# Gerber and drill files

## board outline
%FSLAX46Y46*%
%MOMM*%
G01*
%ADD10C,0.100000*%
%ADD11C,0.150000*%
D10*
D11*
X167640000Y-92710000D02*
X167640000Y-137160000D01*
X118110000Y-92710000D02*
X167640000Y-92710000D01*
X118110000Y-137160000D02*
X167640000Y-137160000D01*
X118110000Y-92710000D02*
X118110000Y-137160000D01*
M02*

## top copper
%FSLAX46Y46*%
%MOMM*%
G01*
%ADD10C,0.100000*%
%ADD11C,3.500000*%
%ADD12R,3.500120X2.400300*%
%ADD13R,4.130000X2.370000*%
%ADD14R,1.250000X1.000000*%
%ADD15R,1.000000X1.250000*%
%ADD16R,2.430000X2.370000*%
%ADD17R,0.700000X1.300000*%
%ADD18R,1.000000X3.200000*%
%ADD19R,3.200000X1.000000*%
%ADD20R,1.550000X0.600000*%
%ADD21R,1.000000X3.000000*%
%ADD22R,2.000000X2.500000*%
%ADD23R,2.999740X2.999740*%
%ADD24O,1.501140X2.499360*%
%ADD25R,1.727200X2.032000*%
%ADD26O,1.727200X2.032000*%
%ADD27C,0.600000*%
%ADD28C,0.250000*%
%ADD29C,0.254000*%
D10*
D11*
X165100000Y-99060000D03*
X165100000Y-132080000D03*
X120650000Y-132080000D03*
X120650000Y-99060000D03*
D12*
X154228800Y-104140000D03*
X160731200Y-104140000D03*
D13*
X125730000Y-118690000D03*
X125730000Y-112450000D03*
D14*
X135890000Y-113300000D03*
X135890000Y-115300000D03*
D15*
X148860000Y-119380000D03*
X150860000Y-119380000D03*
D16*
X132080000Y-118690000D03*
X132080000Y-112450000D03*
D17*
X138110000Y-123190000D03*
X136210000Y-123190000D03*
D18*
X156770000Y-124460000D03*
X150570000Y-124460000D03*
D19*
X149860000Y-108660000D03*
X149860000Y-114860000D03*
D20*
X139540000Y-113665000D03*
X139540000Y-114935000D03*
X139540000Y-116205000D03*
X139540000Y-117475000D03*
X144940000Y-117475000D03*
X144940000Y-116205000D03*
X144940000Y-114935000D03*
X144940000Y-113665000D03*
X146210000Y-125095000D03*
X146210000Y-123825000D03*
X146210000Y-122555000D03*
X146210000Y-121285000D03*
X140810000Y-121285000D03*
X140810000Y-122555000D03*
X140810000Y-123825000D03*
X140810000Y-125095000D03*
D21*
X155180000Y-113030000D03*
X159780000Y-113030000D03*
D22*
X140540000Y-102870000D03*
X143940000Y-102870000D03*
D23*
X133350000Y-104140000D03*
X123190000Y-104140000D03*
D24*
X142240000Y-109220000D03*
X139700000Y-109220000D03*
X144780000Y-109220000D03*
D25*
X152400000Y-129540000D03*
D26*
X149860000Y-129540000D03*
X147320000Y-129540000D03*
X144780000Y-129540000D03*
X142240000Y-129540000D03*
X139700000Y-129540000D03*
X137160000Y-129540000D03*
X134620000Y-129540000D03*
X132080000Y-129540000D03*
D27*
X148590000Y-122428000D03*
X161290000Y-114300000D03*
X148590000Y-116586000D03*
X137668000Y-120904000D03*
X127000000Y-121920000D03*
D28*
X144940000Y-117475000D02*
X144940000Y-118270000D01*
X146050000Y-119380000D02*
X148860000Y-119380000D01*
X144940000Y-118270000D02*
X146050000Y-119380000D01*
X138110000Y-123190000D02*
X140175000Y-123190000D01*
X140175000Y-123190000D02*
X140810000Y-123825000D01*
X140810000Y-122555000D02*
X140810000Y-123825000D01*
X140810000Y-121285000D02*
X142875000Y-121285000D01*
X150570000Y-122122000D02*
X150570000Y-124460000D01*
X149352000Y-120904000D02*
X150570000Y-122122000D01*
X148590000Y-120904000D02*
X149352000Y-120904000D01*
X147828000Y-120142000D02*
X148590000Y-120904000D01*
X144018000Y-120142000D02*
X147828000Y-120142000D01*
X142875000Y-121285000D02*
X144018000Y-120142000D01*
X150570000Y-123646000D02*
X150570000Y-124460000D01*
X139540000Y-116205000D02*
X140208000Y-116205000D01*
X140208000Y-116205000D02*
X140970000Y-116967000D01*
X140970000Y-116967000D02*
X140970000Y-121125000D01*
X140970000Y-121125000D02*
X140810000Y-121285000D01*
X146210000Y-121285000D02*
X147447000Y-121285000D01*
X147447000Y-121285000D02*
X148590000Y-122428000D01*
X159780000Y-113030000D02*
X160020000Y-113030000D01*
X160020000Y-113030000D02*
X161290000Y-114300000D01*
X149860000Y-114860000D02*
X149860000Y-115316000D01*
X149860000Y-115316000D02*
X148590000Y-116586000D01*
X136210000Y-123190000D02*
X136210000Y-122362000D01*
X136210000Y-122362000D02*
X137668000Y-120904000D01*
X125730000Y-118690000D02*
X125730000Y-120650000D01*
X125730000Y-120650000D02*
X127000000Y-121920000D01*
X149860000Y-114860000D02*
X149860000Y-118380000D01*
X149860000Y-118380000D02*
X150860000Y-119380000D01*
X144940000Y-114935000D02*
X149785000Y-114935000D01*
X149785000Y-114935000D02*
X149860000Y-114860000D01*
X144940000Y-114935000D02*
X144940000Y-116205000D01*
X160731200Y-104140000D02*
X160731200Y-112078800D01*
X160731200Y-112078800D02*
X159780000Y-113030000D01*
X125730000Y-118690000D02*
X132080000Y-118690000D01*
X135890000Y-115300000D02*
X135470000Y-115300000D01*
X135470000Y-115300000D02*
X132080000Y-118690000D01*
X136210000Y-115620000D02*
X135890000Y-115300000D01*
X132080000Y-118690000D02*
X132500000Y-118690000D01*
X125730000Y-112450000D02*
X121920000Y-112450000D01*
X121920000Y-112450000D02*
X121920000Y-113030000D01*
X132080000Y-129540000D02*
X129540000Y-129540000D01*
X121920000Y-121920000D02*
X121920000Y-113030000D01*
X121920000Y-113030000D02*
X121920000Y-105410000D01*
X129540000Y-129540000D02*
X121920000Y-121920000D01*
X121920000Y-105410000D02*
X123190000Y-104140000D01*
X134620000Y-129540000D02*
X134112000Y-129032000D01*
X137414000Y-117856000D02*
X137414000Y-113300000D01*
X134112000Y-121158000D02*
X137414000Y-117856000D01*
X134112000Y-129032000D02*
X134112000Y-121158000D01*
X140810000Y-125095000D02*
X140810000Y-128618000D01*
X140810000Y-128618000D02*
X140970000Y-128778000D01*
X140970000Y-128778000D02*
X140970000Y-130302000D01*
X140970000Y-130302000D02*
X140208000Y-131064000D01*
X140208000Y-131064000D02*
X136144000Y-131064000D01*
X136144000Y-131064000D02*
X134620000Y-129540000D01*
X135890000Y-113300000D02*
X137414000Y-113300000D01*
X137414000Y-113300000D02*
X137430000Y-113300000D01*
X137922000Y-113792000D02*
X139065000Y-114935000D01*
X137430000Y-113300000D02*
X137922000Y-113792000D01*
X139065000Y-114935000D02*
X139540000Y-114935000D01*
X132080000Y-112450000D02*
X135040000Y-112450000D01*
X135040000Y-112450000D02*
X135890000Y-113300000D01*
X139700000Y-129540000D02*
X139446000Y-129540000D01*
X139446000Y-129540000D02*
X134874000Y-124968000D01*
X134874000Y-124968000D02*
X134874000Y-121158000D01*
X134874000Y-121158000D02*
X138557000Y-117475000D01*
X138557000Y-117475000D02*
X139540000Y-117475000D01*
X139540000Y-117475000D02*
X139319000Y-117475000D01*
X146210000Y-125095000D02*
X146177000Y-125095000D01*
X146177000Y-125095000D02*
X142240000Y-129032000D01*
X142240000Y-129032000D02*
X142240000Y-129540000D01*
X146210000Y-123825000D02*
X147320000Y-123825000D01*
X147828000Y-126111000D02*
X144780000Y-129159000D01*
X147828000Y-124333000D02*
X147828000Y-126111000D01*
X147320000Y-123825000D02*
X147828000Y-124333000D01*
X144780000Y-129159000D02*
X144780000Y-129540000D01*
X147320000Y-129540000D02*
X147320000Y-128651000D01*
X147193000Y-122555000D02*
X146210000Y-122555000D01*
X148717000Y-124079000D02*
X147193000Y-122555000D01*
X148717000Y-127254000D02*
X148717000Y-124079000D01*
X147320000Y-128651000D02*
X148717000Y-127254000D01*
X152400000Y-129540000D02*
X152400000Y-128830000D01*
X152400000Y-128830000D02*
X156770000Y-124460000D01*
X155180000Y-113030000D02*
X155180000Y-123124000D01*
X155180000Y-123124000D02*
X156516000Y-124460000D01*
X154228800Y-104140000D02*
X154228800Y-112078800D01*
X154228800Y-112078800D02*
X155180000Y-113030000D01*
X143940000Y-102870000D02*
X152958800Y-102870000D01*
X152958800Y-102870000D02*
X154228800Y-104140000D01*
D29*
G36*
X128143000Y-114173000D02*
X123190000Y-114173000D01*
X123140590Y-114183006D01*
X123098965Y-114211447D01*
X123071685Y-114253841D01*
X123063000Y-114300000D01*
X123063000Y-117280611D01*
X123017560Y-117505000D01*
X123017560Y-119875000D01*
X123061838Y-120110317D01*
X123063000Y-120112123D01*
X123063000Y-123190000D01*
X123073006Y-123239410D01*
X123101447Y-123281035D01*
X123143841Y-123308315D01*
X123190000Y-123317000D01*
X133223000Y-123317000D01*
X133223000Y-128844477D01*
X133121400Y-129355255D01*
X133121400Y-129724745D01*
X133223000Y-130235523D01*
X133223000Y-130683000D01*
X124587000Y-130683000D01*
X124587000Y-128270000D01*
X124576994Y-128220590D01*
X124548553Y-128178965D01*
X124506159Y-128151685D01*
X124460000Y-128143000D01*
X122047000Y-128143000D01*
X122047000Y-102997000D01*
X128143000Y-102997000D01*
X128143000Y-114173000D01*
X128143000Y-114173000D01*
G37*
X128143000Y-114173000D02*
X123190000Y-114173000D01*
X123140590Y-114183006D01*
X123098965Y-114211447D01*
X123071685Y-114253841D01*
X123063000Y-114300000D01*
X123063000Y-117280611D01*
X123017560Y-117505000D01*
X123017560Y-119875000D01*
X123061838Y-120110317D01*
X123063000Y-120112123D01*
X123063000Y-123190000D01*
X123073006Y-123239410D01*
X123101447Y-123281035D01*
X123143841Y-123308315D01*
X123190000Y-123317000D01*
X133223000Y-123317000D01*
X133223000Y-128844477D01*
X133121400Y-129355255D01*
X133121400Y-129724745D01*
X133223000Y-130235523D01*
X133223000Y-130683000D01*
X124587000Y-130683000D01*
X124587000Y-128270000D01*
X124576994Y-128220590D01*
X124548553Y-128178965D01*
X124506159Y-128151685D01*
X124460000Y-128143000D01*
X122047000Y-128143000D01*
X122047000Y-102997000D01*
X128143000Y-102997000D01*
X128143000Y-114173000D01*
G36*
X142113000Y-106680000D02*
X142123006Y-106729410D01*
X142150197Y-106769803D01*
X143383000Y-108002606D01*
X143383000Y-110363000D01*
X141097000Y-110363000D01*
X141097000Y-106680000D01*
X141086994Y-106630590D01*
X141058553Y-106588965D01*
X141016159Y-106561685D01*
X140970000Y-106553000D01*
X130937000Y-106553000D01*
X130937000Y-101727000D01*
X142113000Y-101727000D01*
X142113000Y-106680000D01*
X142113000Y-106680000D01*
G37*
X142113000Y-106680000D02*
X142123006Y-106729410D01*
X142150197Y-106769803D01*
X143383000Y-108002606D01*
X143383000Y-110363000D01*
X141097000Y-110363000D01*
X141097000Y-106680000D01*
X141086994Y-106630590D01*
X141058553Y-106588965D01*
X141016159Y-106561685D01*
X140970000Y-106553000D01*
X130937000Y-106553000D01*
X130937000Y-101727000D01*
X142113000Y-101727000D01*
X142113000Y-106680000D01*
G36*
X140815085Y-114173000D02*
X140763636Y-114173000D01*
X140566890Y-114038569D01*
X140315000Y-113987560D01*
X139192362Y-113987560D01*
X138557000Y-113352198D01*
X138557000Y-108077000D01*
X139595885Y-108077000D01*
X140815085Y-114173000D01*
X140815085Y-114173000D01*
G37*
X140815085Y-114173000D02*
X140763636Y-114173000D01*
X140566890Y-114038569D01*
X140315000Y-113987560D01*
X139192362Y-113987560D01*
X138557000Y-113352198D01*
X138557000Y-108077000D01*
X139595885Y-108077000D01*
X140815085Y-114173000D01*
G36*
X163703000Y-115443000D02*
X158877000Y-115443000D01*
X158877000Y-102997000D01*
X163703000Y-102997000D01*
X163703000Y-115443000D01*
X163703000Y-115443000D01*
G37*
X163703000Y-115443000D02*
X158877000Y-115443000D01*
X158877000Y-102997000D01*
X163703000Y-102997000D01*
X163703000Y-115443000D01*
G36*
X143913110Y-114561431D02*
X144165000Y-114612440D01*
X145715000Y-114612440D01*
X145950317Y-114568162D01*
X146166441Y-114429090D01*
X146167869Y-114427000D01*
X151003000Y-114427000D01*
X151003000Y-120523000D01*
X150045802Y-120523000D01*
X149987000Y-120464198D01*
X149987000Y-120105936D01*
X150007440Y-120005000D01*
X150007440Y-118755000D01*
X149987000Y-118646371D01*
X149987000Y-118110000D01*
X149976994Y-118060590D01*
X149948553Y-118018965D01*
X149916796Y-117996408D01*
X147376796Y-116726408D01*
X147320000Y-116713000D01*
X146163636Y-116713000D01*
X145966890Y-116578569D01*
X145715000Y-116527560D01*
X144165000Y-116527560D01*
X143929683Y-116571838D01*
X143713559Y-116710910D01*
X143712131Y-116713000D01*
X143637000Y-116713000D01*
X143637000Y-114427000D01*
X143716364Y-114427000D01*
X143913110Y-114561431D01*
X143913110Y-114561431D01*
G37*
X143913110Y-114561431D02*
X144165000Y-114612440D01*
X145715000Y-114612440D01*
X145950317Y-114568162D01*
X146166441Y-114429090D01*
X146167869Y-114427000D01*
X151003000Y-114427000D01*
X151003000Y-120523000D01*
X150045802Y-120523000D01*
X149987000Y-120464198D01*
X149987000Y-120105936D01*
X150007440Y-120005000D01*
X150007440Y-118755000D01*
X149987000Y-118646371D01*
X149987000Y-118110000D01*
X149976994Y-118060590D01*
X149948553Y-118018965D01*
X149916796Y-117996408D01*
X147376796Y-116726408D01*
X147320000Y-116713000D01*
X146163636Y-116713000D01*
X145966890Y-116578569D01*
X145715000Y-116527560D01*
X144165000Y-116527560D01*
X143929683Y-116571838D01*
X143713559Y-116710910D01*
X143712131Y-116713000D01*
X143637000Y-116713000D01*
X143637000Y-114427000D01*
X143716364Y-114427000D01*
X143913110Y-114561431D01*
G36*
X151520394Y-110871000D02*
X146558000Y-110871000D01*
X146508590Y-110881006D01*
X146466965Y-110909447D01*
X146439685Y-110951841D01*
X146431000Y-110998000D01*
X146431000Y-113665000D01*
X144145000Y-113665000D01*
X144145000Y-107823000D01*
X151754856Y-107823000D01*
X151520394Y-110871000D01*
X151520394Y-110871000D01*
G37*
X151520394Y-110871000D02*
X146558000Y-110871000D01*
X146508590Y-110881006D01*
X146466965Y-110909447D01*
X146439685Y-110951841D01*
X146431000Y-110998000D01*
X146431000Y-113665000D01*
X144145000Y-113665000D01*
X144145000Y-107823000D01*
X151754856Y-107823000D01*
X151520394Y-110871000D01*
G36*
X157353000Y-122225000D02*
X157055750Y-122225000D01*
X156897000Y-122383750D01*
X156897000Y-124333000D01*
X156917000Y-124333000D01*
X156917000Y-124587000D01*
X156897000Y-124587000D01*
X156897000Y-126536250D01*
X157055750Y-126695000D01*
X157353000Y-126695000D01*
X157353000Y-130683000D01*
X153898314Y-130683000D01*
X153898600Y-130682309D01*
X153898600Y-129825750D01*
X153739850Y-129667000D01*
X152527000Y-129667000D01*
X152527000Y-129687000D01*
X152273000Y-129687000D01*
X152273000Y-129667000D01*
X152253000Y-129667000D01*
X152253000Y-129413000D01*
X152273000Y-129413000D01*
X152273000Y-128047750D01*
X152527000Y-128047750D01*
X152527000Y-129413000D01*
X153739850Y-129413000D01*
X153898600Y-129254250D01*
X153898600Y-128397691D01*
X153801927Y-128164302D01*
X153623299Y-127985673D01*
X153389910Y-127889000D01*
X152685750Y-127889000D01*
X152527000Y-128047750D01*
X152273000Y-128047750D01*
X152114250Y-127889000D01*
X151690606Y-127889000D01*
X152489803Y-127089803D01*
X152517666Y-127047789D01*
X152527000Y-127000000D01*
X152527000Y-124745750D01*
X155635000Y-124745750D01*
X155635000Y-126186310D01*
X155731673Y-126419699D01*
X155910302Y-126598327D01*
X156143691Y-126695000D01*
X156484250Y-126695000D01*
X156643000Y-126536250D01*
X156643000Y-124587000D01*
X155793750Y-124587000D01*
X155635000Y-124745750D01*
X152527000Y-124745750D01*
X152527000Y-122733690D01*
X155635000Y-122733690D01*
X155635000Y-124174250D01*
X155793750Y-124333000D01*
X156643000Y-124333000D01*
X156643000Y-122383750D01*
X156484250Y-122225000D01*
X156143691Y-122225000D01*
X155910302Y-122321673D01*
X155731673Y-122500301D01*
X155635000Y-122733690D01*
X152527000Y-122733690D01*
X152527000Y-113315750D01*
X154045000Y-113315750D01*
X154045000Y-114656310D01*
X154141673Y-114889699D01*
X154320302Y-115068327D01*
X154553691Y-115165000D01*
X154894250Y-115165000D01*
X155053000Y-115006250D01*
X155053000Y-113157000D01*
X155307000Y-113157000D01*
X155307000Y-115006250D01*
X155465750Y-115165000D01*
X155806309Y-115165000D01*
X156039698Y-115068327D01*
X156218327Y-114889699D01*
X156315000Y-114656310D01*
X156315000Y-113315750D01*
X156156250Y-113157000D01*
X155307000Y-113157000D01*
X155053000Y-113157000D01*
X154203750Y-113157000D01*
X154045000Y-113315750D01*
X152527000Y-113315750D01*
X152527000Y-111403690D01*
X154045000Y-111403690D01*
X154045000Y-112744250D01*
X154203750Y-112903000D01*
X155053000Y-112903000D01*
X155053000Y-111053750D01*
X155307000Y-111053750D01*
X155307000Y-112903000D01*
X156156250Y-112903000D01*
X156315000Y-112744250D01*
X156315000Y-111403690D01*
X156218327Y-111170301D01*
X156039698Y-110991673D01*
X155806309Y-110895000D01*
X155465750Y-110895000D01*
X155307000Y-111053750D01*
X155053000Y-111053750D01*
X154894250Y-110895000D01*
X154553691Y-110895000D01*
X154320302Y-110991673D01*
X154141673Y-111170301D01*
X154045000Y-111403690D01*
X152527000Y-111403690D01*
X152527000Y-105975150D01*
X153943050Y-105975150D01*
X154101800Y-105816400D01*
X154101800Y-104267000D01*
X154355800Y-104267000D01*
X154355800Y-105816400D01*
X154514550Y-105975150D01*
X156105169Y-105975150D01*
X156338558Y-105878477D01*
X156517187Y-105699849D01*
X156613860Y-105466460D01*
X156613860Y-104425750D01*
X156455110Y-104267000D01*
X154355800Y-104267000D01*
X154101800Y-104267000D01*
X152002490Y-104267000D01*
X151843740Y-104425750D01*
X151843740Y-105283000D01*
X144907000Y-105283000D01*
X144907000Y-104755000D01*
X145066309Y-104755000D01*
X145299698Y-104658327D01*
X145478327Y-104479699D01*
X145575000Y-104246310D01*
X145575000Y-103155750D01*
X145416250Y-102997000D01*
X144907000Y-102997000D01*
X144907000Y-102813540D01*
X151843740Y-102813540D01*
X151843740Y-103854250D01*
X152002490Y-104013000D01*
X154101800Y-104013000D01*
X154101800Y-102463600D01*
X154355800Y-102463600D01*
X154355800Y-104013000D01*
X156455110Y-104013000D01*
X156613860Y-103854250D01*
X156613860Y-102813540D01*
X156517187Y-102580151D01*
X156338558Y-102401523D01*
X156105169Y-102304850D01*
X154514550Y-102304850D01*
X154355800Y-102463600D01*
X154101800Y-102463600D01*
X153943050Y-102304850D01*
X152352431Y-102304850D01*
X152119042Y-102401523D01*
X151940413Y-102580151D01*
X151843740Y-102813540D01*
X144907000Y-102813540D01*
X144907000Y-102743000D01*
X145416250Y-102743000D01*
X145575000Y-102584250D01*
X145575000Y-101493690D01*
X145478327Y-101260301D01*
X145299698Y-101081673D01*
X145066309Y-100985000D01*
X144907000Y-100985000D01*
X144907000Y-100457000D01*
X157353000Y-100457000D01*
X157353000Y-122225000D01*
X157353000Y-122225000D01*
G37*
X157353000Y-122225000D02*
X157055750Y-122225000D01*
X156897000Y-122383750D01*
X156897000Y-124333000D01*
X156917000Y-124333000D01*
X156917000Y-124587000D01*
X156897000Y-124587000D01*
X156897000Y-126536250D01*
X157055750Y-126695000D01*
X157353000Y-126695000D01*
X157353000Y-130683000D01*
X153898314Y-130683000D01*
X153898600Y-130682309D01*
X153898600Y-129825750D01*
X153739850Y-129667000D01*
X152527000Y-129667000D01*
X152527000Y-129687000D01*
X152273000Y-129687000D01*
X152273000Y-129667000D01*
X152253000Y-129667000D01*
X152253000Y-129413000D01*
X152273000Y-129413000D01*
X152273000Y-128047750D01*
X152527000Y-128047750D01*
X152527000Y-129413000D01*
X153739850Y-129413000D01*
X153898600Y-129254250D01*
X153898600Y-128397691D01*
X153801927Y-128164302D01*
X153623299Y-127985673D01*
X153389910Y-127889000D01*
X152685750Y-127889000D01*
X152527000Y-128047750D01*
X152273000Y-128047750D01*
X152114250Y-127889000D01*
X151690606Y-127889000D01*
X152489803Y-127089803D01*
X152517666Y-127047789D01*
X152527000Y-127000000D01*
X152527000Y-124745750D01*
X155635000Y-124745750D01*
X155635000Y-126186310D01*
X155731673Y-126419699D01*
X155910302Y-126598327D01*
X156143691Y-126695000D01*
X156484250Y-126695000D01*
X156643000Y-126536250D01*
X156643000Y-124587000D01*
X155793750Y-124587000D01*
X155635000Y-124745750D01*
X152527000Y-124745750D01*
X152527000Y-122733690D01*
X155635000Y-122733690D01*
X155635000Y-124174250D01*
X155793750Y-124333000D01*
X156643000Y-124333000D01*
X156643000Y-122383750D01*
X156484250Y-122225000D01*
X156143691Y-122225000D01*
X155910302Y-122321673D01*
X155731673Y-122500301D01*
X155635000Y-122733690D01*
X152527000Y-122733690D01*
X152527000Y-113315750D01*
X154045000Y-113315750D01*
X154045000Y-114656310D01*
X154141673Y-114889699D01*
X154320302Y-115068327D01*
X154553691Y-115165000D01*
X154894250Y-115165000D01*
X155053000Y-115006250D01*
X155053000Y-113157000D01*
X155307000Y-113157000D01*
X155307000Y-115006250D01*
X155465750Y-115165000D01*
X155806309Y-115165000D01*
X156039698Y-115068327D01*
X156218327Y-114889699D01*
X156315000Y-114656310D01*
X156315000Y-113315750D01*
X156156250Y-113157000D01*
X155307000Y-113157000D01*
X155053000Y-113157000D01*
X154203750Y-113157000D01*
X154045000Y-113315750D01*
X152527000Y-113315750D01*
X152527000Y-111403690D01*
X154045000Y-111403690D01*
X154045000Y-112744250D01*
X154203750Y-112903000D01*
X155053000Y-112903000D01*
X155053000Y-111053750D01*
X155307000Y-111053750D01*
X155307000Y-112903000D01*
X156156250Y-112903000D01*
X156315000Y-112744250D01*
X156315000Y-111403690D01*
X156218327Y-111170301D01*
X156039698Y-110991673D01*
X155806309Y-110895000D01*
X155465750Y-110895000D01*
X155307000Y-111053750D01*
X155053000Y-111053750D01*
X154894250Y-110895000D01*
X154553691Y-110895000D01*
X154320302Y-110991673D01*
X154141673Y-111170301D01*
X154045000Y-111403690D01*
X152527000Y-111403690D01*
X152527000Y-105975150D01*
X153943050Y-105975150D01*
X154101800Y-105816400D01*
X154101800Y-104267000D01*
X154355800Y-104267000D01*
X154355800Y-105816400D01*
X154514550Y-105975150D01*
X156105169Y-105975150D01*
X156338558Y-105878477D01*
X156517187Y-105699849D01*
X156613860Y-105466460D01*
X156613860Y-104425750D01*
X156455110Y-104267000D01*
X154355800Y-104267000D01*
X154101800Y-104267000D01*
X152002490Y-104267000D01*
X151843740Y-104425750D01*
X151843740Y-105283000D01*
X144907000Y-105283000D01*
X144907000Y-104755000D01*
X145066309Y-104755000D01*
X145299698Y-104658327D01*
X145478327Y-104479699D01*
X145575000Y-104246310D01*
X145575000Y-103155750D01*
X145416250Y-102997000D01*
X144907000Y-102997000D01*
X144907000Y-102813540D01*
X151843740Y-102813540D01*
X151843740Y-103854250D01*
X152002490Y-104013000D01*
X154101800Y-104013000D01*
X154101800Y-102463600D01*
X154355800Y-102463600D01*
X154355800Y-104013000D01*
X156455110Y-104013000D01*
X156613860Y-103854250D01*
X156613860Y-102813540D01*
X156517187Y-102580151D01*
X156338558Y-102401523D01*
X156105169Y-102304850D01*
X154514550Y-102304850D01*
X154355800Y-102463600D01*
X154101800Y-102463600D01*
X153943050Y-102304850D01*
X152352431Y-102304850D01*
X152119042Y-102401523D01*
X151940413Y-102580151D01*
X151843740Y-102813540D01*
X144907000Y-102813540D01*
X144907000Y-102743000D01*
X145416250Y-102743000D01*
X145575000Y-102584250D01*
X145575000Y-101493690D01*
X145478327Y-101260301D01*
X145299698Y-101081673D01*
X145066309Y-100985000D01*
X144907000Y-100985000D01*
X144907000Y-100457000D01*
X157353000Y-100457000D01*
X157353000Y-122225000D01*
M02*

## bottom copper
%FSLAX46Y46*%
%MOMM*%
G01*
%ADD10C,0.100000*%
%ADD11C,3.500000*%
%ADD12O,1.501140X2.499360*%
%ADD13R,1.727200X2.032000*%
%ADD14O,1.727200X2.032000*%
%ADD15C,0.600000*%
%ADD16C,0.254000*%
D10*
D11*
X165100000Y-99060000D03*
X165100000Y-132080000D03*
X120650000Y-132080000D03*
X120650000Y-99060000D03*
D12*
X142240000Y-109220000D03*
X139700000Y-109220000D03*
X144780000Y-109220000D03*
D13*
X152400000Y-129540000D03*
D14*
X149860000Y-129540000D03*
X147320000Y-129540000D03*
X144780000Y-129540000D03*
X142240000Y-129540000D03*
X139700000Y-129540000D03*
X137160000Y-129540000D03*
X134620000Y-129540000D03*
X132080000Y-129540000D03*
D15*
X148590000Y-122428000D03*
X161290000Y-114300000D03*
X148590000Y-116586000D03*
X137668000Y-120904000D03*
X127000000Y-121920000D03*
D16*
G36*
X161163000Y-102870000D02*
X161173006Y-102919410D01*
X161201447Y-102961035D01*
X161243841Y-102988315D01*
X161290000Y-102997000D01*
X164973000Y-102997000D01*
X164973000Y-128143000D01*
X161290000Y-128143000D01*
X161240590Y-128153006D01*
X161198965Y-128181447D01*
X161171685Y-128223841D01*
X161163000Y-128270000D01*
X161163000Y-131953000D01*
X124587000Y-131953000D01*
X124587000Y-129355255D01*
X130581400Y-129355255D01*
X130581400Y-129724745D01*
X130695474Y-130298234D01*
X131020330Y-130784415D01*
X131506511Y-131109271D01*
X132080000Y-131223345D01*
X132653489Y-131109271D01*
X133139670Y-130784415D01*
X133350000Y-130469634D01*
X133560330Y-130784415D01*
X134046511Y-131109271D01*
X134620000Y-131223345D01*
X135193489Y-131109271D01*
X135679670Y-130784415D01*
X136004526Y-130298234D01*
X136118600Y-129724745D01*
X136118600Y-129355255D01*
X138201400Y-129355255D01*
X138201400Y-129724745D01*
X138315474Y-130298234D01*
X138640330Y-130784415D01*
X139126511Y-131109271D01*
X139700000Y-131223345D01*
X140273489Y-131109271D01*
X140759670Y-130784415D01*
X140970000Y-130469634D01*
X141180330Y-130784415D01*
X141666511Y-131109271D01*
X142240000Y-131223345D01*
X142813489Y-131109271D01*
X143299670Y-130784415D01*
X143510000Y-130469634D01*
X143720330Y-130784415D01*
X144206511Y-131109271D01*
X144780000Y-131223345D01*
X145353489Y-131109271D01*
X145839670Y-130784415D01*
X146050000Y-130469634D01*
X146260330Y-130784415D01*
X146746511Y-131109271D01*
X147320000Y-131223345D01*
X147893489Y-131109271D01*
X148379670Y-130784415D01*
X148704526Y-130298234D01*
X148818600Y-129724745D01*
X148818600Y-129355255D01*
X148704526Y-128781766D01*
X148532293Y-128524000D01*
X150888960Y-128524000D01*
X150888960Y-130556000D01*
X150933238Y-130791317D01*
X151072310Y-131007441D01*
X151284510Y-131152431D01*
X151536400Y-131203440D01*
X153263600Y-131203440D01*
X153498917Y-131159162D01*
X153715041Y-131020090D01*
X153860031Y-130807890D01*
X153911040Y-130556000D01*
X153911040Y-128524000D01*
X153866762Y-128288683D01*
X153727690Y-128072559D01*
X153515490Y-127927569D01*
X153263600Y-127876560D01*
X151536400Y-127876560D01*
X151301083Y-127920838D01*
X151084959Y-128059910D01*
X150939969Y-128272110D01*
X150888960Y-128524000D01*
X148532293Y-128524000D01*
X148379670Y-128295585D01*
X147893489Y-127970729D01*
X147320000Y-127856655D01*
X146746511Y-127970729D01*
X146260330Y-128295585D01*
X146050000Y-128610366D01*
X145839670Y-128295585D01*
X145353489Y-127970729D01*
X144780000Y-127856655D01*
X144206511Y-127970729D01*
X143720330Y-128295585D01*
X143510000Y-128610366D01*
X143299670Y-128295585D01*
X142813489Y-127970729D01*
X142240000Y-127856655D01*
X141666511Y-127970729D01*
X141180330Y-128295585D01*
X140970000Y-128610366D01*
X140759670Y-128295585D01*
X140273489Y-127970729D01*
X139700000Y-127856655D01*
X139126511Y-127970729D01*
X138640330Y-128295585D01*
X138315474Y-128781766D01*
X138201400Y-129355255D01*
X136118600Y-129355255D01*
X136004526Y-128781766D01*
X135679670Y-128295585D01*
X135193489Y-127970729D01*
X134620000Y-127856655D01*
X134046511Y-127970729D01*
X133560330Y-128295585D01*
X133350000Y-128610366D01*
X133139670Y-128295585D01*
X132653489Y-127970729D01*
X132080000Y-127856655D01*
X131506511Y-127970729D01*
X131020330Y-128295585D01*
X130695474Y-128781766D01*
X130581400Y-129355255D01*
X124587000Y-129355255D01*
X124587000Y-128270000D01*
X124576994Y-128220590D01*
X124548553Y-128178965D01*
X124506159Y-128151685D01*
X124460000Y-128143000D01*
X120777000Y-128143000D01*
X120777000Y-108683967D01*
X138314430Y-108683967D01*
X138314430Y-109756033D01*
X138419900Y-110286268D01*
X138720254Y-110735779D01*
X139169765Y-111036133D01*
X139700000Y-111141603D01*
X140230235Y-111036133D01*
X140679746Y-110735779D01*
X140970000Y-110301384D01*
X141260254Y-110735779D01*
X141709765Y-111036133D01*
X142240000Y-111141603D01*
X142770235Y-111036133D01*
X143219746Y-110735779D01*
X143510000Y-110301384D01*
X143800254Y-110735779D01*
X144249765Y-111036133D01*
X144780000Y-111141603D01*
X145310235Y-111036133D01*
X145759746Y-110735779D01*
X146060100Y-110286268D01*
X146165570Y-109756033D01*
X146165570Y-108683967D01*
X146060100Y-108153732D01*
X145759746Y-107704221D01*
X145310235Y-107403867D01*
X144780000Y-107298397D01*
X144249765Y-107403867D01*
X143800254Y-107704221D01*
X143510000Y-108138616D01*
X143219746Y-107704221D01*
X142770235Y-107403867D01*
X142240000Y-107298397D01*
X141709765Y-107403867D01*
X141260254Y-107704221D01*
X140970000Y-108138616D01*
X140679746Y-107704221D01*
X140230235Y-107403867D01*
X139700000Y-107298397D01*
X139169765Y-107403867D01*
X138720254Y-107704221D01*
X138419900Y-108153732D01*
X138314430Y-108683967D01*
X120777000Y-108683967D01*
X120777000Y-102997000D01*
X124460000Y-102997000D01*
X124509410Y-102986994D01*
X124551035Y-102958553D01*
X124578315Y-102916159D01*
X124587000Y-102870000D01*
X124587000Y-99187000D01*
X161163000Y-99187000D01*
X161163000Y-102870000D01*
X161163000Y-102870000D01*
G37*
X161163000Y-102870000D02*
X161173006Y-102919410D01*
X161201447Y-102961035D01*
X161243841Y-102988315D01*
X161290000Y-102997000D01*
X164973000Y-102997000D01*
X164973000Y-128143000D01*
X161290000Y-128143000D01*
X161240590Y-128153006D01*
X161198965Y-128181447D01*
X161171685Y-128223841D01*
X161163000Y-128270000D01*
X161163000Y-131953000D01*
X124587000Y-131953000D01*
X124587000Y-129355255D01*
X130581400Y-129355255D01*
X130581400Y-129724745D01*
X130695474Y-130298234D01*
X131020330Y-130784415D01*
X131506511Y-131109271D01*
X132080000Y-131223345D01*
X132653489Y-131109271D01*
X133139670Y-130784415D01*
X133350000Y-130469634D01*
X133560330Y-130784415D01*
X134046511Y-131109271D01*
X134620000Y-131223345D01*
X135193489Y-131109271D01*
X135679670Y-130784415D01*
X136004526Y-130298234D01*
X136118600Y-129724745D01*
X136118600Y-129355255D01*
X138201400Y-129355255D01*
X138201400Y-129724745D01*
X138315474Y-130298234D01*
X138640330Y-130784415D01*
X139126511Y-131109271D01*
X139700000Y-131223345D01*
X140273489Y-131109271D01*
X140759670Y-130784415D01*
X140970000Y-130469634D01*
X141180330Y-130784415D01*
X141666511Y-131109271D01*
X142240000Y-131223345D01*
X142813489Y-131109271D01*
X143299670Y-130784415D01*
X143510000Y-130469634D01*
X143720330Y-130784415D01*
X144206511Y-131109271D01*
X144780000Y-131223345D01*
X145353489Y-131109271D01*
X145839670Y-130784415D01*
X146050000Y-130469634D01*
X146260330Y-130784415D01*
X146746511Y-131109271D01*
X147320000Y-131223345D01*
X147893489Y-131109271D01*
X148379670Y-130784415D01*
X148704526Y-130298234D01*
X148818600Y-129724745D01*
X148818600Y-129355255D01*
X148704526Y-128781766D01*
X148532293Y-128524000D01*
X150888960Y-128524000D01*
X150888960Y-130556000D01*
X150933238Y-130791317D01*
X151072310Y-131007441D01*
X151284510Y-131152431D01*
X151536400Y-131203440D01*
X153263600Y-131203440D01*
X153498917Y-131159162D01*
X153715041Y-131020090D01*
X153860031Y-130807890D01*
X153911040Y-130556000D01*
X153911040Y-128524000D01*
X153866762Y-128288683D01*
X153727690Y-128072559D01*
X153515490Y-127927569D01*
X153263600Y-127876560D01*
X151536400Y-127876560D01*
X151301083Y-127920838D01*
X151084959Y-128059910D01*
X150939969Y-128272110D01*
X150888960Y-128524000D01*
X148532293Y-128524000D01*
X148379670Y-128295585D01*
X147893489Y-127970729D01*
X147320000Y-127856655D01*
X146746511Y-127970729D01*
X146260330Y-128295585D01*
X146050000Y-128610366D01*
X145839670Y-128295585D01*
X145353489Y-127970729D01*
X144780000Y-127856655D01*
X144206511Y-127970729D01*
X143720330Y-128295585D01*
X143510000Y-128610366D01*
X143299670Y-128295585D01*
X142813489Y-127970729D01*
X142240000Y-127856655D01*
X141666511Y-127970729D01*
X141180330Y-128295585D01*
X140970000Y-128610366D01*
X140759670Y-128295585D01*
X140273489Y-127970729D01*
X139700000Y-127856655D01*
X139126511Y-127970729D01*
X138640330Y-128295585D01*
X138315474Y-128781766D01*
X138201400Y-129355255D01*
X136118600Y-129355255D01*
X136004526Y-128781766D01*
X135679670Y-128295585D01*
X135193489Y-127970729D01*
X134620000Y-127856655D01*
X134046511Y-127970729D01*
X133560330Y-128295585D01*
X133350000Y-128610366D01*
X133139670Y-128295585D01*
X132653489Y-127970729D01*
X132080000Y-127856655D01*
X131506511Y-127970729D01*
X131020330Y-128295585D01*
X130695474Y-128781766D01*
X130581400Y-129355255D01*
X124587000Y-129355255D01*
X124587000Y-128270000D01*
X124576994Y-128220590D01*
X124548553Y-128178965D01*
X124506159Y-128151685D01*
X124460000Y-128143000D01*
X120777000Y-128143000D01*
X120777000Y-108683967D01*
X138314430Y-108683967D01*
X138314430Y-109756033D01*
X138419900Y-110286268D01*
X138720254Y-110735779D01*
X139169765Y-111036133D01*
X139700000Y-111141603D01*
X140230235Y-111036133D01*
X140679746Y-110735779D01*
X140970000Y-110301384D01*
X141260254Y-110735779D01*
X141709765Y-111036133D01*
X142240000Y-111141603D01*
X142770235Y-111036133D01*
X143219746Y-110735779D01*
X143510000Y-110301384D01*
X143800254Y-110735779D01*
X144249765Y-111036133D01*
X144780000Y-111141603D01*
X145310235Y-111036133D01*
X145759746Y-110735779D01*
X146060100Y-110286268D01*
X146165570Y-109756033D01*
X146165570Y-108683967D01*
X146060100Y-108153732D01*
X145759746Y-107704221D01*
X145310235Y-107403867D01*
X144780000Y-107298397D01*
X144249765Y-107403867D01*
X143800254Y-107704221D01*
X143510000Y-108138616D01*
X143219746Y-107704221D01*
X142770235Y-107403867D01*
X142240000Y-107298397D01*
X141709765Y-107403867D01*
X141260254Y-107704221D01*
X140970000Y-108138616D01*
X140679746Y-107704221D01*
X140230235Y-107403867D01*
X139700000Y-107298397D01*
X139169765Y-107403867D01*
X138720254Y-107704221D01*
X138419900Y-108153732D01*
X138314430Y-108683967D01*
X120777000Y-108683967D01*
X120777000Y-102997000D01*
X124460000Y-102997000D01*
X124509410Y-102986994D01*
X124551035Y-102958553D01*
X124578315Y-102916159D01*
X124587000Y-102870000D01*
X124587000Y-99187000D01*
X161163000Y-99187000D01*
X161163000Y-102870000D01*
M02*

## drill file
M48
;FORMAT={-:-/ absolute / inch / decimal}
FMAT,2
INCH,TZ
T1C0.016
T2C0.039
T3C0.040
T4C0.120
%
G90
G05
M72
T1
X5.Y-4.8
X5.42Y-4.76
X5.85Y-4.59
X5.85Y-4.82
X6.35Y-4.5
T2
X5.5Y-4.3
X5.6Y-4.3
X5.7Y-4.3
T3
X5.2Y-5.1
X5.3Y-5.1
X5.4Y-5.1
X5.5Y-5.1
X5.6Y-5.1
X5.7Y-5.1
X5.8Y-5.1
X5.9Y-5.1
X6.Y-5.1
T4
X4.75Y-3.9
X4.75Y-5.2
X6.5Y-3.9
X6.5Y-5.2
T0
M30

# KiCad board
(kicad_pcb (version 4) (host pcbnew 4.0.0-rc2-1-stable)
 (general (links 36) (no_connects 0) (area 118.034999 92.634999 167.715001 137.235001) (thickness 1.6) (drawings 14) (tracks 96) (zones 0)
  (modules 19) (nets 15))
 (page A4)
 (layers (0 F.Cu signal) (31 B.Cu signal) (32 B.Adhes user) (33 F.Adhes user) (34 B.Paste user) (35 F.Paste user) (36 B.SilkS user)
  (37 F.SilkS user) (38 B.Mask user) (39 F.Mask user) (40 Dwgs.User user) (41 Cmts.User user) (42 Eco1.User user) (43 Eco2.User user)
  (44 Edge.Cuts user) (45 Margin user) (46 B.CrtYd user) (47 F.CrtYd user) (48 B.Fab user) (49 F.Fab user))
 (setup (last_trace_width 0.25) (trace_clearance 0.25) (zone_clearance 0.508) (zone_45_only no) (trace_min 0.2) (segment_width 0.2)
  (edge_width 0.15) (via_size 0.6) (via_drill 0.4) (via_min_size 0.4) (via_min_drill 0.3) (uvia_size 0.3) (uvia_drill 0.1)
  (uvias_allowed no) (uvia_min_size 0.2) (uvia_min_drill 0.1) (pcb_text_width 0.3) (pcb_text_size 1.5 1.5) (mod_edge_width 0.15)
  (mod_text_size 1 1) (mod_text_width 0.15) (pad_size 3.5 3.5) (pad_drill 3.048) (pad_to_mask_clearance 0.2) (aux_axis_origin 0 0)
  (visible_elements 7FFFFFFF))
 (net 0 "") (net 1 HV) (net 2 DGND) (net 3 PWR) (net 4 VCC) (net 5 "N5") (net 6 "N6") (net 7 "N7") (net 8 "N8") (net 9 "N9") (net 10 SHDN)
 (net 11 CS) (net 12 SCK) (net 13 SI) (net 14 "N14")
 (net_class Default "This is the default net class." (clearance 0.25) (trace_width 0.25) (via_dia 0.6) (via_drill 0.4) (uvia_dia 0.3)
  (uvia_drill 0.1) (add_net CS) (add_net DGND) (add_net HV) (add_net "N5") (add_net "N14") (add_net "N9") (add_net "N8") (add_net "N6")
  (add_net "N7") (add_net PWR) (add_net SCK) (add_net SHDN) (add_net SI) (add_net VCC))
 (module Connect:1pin (layer F.Cu) (at 165.1 99.06)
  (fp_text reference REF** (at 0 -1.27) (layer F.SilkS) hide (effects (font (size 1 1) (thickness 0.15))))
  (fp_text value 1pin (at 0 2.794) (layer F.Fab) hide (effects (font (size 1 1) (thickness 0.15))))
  (pad 1 thru_hole circle (at 0 0) (size 3.5 3.5) (drill 3.048) (layers *.Cu *.Mask F.SilkS)))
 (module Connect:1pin (layer F.Cu) (at 165.1 132.08)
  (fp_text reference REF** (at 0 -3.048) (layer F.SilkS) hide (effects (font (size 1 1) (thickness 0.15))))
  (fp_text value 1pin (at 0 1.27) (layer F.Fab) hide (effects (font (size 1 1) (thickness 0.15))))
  (pad 1 thru_hole circle (at 0 0) (size 3.5 3.5) (drill 3.048) (layers *.Cu *.Mask F.SilkS)))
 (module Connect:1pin (layer F.Cu) (at 120.65 132.08)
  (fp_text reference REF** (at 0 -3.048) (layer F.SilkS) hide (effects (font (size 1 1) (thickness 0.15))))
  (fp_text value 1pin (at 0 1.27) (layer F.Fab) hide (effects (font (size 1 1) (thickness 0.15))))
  (pad 1 thru_hole circle (at 0 0) (size 3.5 3.5) (drill 3.048) (layers *.Cu *.Mask F.SilkS)))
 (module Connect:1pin (layer F.Cu) (at 120.65 99.06)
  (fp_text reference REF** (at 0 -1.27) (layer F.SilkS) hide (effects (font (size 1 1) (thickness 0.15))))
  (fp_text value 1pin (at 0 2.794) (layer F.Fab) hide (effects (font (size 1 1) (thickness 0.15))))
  (pad 1 thru_hole circle (at 0 0) (size 3.5 3.5) (drill 3.048) (layers *.Cu *.Mask F.SilkS)))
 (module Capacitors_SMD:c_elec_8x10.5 (layer F.Cu) (at 157.48 104.14 180)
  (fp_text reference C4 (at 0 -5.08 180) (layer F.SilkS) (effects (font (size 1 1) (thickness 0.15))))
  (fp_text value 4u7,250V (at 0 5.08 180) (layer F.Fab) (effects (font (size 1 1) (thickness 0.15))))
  (pad 1 smd rect (at 3.2512 0 180) (size 3.50012 2.4003) (layers F.Cu F.Paste F.Mask) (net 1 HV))
  (pad 2 smd rect (at -3.2512 0 180) (size 3.50012 2.4003) (layers F.Cu F.Paste F.Mask) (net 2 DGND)))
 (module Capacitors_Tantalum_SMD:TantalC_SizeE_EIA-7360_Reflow (layer F.Cu) (at 125.73 115.57 270)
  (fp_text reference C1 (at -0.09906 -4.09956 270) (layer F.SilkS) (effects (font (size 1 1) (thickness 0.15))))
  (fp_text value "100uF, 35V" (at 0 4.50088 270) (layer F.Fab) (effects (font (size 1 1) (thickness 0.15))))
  (pad 2 smd rect (at 3.12 0 270) (size 2.37 4.13) (layers F.Cu F.Paste F.Mask) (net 2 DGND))
  (pad 1 smd rect (at -3.12 0 270) (size 2.37 4.13) (layers F.Cu F.Paste F.Mask) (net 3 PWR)))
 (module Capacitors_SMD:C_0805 (layer F.Cu) (at 135.89 114.3 270)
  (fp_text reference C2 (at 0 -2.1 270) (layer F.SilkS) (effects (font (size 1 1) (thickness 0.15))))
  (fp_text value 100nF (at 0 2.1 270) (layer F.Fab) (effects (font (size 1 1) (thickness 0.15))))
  (pad 1 smd rect (at -1 0 270) (size 1 1.25) (layers F.Cu F.Paste F.Mask) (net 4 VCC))
  (pad 2 smd rect (at 1 0 270) (size 1 1.25) (layers F.Cu F.Paste F.Mask) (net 2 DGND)))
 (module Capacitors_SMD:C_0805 (layer F.Cu) (at 149.86 119.38)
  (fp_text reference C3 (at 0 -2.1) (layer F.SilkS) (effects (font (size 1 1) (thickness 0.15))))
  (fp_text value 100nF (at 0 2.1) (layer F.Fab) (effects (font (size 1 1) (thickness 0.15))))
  (pad 1 smd rect (at -1 0) (size 1 1.25) (layers F.Cu F.Paste F.Mask) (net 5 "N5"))
  (pad 2 smd rect (at 1 0) (size 1 1.25) (layers F.Cu F.Paste F.Mask) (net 2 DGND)))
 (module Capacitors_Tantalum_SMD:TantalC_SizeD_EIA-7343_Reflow (layer F.Cu) (at 132.08 115.57 270)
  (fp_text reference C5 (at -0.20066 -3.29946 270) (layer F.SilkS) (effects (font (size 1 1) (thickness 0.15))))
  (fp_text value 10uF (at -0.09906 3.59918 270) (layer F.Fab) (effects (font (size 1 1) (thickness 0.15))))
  (pad 2 smd rect (at 3.12 0 270) (size 2.37 2.43) (layers F.Cu F.Paste F.Mask) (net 2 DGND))
  (pad 1 smd rect (at -3.12 0 270) (size 2.37 2.43) (layers F.Cu F.Paste F.Mask) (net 4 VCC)))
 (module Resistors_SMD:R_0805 (layer F.Cu) (at 137.16 123.19 180)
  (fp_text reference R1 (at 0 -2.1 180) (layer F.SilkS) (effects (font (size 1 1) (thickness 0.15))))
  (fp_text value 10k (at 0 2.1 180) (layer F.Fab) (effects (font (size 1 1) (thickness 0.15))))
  (pad 1 smd rect (at -0.95 0 180) (size 0.7 1.3) (layers F.Cu F.Paste F.Mask) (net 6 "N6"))
  (pad 2 smd rect (at 0.95 0 180) (size 0.7 1.3) (layers F.Cu F.Paste F.Mask) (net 2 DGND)))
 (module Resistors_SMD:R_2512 (layer F.Cu) (at 153.67 124.46 180)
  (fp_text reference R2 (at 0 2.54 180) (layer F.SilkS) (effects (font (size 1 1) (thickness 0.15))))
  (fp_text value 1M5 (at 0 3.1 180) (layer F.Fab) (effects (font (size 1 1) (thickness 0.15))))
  (pad 1 smd rect (at -3.1 0 180) (size 1 3.2) (layers F.Cu F.Paste F.Mask) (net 1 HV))
  (pad 2 smd rect (at 3.1 0 180) (size 1 3.2) (layers F.Cu F.Paste F.Mask) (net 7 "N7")))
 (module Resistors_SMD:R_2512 (layer F.Cu) (at 149.86 111.76 270)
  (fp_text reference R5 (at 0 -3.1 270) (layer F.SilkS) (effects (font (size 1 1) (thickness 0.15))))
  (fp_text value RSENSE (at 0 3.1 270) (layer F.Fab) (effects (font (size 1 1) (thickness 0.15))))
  (pad 1 smd rect (at -3.1 0 270) (size 1 3.2) (layers F.Cu F.Paste F.Mask) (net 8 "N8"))
  (pad 2 smd rect (at 3.1 0 270) (size 1 3.2) (layers F.Cu F.Paste F.Mask) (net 2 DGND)))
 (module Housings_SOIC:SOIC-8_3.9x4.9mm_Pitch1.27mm (layer F.Cu) (at 142.24 115.57)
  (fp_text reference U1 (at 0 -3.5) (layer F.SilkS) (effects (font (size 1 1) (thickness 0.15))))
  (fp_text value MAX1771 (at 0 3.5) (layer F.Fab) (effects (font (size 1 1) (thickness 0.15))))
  (pad 1 smd rect (at -2.7 -1.905) (size 1.55 0.6) (layers F.Cu F.Paste F.Mask) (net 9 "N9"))
  (pad 2 smd rect (at -2.7 -0.635) (size 1.55 0.6) (layers F.Cu F.Paste F.Mask) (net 4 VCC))
  (pad 3 smd rect (at -2.7 0.635) (size 1.55 0.6) (layers F.Cu F.Paste F.Mask) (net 7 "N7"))
  (pad 4 smd rect (at -2.7 1.905) (size 1.55 0.6) (layers F.Cu F.Paste F.Mask) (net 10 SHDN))
  (pad 5 smd rect (at 2.7 1.905) (size 1.55 0.6) (layers F.Cu F.Paste F.Mask) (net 5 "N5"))
  (pad 6 smd rect (at 2.7 0.635) (size 1.55 0.6) (layers F.Cu F.Paste F.Mask) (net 2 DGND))
  (pad 7 smd rect (at 2.7 -0.635) (size 1.55 0.6) (layers F.Cu F.Paste F.Mask) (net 2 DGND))
  (pad 8 smd rect (at 2.7 -1.905) (size 1.55 0.6) (layers F.Cu F.Paste F.Mask) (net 8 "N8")))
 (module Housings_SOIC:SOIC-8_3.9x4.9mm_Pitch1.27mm (layer F.Cu) (at 143.51 123.19 180)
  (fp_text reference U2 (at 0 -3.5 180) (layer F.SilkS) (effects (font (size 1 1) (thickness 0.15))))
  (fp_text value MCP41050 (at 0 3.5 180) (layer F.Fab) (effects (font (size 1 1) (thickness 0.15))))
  (pad 1 smd rect (at -2.7 -1.905 180) (size 1.55 0.6) (layers F.Cu F.Paste F.Mask) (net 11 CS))
  (pad 2 smd rect (at -2.7 -0.635 180) (size 1.55 0.6) (layers F.Cu F.Paste F.Mask) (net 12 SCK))
  (pad 3 smd rect (at -2.7 0.635 180) (size 1.55 0.6) (layers F.Cu F.Paste F.Mask) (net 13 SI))
  (pad 4 smd rect (at -2.7 1.905 180) (size 1.55 0.6) (layers F.Cu F.Paste F.Mask) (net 2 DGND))
  (pad 5 smd rect (at 2.7 1.905 180) (size 1.55 0.6) (layers F.Cu F.Paste F.Mask) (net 7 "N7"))
  (pad 6 smd rect (at 2.7 0.635 180) (size 1.55 0.6) (layers F.Cu F.Paste F.Mask) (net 6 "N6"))
  (pad 7 smd rect (at 2.7 -0.635 180) (size 1.55 0.6) (layers F.Cu F.Paste F.Mask) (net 6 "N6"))
  (pad 8 smd rect (at 2.7 -1.905 180) (size 1.55 0.6) (layers F.Cu F.Paste F.Mask) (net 4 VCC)))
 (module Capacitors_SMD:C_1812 (layer F.Cu) (at 157.48 113.03)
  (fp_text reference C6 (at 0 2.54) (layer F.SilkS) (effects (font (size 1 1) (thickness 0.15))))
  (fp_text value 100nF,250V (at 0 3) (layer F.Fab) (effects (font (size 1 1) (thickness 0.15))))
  (pad 1 smd rect (at -2.3 0) (size 1 3) (layers F.Cu F.Paste F.Mask) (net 1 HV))
  (pad 2 smd rect (at 2.3 0) (size 1 3) (layers F.Cu F.Paste F.Mask) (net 2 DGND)))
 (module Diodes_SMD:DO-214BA (layer F.Cu) (at 142.24 102.87 180)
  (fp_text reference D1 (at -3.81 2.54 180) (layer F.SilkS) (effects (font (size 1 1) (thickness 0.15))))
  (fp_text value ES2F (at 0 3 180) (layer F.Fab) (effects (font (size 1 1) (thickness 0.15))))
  (pad 2 smd rect (at 1.7 0 180) (size 2 2.5) (layers F.Cu F.Paste F.Mask) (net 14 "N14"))
  (pad 1 smd rect (at -1.7 0 180) (size 2 2.5) (layers F.Cu F.Paste F.Mask) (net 1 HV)))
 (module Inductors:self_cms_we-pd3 (layer F.Cu) (at 128.27 104.14 180)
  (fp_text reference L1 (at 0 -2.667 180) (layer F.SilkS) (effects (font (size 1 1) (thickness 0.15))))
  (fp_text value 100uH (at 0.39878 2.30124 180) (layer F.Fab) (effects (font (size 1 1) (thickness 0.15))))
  (pad 1 smd rect (at -5.08 0 180) (size 2.99974 2.99974) (layers F.Cu F.Paste F.Mask) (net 14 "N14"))
  (pad 2 smd rect (at 5.08 0 180) (size 2.99974 2.99974) (layers F.Cu F.Paste F.Mask) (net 3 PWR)))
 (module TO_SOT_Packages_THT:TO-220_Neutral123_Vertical (layer F.Cu) (at 142.24 109.22)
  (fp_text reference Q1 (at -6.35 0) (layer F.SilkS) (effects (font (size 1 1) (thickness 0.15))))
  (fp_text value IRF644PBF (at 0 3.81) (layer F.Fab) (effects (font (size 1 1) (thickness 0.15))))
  (pad 2 thru_hole oval (at 0 0 90) (size 2.49936 1.50114) (drill 1.00076) (layers *.Cu *.Mask F.SilkS) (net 14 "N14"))
  (pad 1 thru_hole oval (at -2.54 0 90) (size 2.49936 1.50114) (drill 1.00076) (layers *.Cu *.Mask F.SilkS) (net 9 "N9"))
  (pad 3 thru_hole oval (at 2.54 0 90) (size 2.49936 1.50114) (drill 1.00076) (layers *.Cu *.Mask F.SilkS) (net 8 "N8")))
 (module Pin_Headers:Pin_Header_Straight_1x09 (layer F.Cu) (at 152.4 129.54 270)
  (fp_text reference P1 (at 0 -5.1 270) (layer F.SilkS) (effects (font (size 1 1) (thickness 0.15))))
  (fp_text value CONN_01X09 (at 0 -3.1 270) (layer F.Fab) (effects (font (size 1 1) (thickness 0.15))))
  (pad 1 thru_hole rect (at 0 0 270) (size 2.032 1.7272) (drill 1.016) (layers *.Cu *.Mask F.SilkS) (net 1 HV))
  (pad 2 thru_hole oval (at 0 2.54 270) (size 2.032 1.7272) (drill 1.016) (layers *.Cu *.Mask F.SilkS) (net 2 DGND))
  (pad 3 thru_hole oval (at 0 5.08 270) (size 2.032 1.7272) (drill 1.016) (layers *.Cu *.Mask F.SilkS) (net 13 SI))
  (pad 4 thru_hole oval (at 0 7.62 270) (size 2.032 1.7272) (drill 1.016) (layers *.Cu *.Mask F.SilkS) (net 12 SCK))
  (pad 5 thru_hole oval (at 0 10.16 270) (size 2.032 1.7272) (drill 1.016) (layers *.Cu *.Mask F.SilkS) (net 11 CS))
  (pad 6 thru_hole oval (at 0 12.7 270) (size 2.032 1.7272) (drill 1.016) (layers *.Cu *.Mask F.SilkS) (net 10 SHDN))
  (pad 7 thru_hole oval (at 0 15.24 270) (size 2.032 1.7272) (drill 1.016) (layers *.Cu *.Mask F.SilkS) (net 2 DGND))
  (pad 8 thru_hole oval (at 0 17.78 270) (size 2.032 1.7272) (drill 1.016) (layers *.Cu *.Mask F.SilkS) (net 4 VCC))
  (pad 9 thru_hole oval (at 0 20.32 270) (size 2.032 1.7272) (drill 1.016) (layers *.Cu *.Mask F.SilkS) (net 3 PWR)))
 (gr_line (start 167.64 92.71) (end 167.64 137.16) (angle 90) (layer Edge.Cuts) (width 0.15))
 (gr_line (start 118.11 92.71) (end 167.64 92.71) (angle 90) (layer Edge.Cuts) (width 0.15))
 (gr_line (start 118.11 137.16) (end 167.64 137.16) (angle 90) (layer Edge.Cuts) (width 0.15))
 (gr_line (start 118.11 92.71) (end 118.11 137.16) (angle 90) (layer Edge.Cuts) (width 0.15))
 (segment (start 144.94 117.475) (end 144.94 118.27) (width 0.25) (layer F.Cu) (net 5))
 (segment (start 146.05 119.38) (end 148.86 119.38) (width 0.25) (layer F.Cu) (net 5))
 (segment (start 144.94 118.27) (end 146.05 119.38) (width 0.25) (layer F.Cu) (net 5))
 (segment (start 138.11 123.19) (end 140.175 123.19) (width 0.25) (layer F.Cu) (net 6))
 (segment (start 140.175 123.19) (end 140.81 123.825) (width 0.25) (layer F.Cu) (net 6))
 (segment (start 140.81 122.555) (end 140.81 123.825) (width 0.25) (layer F.Cu) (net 6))
 (segment (start 140.81 121.285) (end 142.875 121.285) (width 0.25) (layer F.Cu) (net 7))
 (segment (start 150.57 122.122) (end 150.57 124.46) (width 0.25) (layer F.Cu) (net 7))
 (segment (start 149.352 120.904) (end 150.57 122.122) (width 0.25) (layer F.Cu) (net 7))
 (segment (start 148.59 120.904) (end 149.352 120.904) (width 0.25) (layer F.Cu) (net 7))
 (segment (start 147.828 120.142) (end 148.59 120.904) (width 0.25) (layer F.Cu) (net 7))
 (segment (start 144.018 120.142) (end 147.828 120.142) (width 0.25) (layer F.Cu) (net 7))
 (segment (start 142.875 121.285) (end 144.018 120.142) (width 0.25) (layer F.Cu) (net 7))
 (segment (start 150.57 123.646) (end 150.57 124.46) (width 0.25) (layer F.Cu) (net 7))
 (segment (start 139.54 116.205) (end 140.208 116.205) (width 0.25) (layer F.Cu) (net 7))
 (segment (start 140.208 116.205) (end 140.97 116.967) (width 0.25) (layer F.Cu) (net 7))
 (segment (start 140.97 116.967) (end 140.97 121.125) (width 0.25) (layer F.Cu) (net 7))
 (segment (start 140.97 121.125) (end 140.81 121.285) (width 0.25) (layer F.Cu) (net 7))
 (segment (start 146.21 121.285) (end 147.447 121.285) (width 0.25) (layer F.Cu) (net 2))
 (via (at 148.59 122.428) (size 0.6) (drill 0.4) (layers F.Cu B.Cu) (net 2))
 (segment (start 147.447 121.285) (end 148.59 122.428) (width 0.25) (layer F.Cu) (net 2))
 (segment (start 159.78 113.03) (end 160.02 113.03) (width 0.25) (layer F.Cu) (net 2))
 (segment (start 160.02 113.03) (end 161.29 114.3) (width 0.25) (layer F.Cu) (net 2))
 (via (at 161.29 114.3) (size 0.6) (drill 0.4) (layers F.Cu B.Cu) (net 2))
 (segment (start 149.86 114.86) (end 149.86 115.316) (width 0.25) (layer F.Cu) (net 2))
 (segment (start 149.86 115.316) (end 148.59 116.586) (width 0.25) (layer F.Cu) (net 2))
 (via (at 148.59 116.586) (size 0.6) (drill 0.4) (layers F.Cu B.Cu) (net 2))
 (segment (start 136.21 123.19) (end 136.21 122.362) (width 0.25) (layer F.Cu) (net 2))
 (via (at 137.668 120.904) (size 0.6) (drill 0.4) (layers F.Cu B.Cu) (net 2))
 (segment (start 136.21 122.362) (end 137.668 120.904) (width 0.25) (layer F.Cu) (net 2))
 (segment (start 125.73 118.69) (end 125.73 120.65) (width 0.25) (layer F.Cu) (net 2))
 (via (at 127 121.92) (size 0.6) (drill 0.4) (layers F.Cu B.Cu) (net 2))
 (segment (start 125.73 120.65) (end 127 121.92) (width 0.25) (layer F.Cu) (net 2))
 (segment (start 149.86 114.86) (end 149.86 118.38) (width 0.25) (layer F.Cu) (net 2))
 (segment (start 149.86 118.38) (end 150.86 119.38) (width 0.25) (layer F.Cu) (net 2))
 (segment (start 144.94 114.935) (end 149.785 114.935) (width 0.25) (layer F.Cu) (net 2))
 (segment (start 149.785 114.935) (end 149.86 114.86) (width 0.25) (layer F.Cu) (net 2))
 (segment (start 144.94 114.935) (end 144.94 116.205) (width 0.25) (layer F.Cu) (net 2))
 (segment (start 160.7312 104.14) (end 160.7312 112.0788) (width 0.25) (layer F.Cu) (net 2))
 (segment (start 160.7312 112.0788) (end 159.78 113.03) (width 0.25) (layer F.Cu) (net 2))
 (segment (start 125.73 118.69) (end 132.08 118.69) (width 0.25) (layer F.Cu) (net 2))
 (segment (start 135.89 115.3) (end 135.47 115.3) (width 0.25) (layer F.Cu) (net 2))
 (segment (start 135.47 115.3) (end 132.08 118.69) (width 0.25) (layer F.Cu) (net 2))
 (segment (start 136.21 115.62) (end 135.89 115.3) (width 0.25) (layer F.Cu) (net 2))
 (segment (start 132.08 118.69) (end 132.5 118.69) (width 0.25) (layer F.Cu) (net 2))
 (segment (start 125.73 112.45) (end 121.92 112.45) (width 0.25) (layer F.Cu) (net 3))
 (segment (start 121.92 112.45) (end 121.92 113.03) (width 0.25) (layer F.Cu) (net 3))
 (segment (start 132.08 129.54) (end 129.54 129.54) (width 0.25) (layer F.Cu) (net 3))
 (segment (start 121.92 121.92) (end 121.92 113.03) (width 0.25) (layer F.Cu) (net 3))
 (segment (start 121.92 113.03) (end 121.92 105.41) (width 0.25) (layer F.Cu) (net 3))
 (segment (start 129.54 129.54) (end 121.92 121.92) (width 0.25) (layer F.Cu) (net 3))
 (segment (start 121.92 105.41) (end 123.19 104.14) (width 0.25) (layer F.Cu) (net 3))
 (segment (start 134.62 129.54) (end 134.112 129.032) (width 0.25) (layer F.Cu) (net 4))
 (segment (start 137.414 117.856) (end 137.414 113.3) (width 0.25) (layer F.Cu) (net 4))
 (segment (start 134.112 121.158) (end 137.414 117.856) (width 0.25) (layer F.Cu) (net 4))
 (segment (start 134.112 129.032) (end 134.112 121.158) (width 0.25) (layer F.Cu) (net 4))
 (segment (start 140.81 125.095) (end 140.81 128.618) (width 0.25) (layer F.Cu) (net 4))
 (segment (start 140.81 128.618) (end 140.97 128.778) (width 0.25) (layer F.Cu) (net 4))
 (segment (start 140.97 128.778) (end 140.97 130.302) (width 0.25) (layer F.Cu) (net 4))
 (segment (start 140.97 130.302) (end 140.208 131.064) (width 0.25) (layer F.Cu) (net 4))
 (segment (start 140.208 131.064) (end 136.144 131.064) (width 0.25) (layer F.Cu) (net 4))
 (segment (start 136.144 131.064) (end 134.62 129.54) (width 0.25) (layer F.Cu) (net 4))
 (segment (start 135.89 113.3) (end 137.414 113.3) (width 0.25) (layer F.Cu) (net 4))
 (segment (start 137.414 113.3) (end 137.43 113.3) (width 0.25) (layer F.Cu) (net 4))
 (segment (start 137.922 113.792) (end 139.065 114.935) (width 0.25) (layer F.Cu) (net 4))
 (segment (start 137.43 113.3) (end 137.922 113.792) (width 0.25) (layer F.Cu) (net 4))
 (segment (start 139.065 114.935) (end 139.54 114.935) (width 0.25) (layer F.Cu) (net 4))
 (segment (start 132.08 112.45) (end 135.04 112.45) (width 0.25) (layer F.Cu) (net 4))
 (segment (start 135.04 112.45) (end 135.89 113.3) (width 0.25) (layer F.Cu) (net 4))
 (segment (start 139.7 129.54) (end 139.446 129.54) (width 0.25) (layer F.Cu) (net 10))
 (segment (start 139.446 129.54) (end 134.874 124.968) (width 0.25) (layer F.Cu) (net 10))
 (segment (start 134.874 124.968) (end 134.874 121.158) (width 0.25) (layer F.Cu) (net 10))
 (segment (start 134.874 121.158) (end 138.557 117.475) (width 0.25) (layer F.Cu) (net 10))
 (segment (start 138.557 117.475) (end 139.54 117.475) (width 0.25) (layer F.Cu) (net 10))
 (segment (start 139.54 117.475) (end 139.319 117.475) (width 0.25) (layer F.Cu) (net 10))
 (segment (start 146.21 125.095) (end 146.177 125.095) (width 0.25) (layer F.Cu) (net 11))
 (segment (start 146.177 125.095) (end 142.24 129.032) (width 0.25) (layer F.Cu) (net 11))
 (segment (start 142.24 129.032) (end 142.24 129.54) (width 0.25) (layer F.Cu) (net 11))
 (segment (start 146.21 123.825) (end 147.32 123.825) (width 0.25) (layer F.Cu) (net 12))
 (segment (start 147.828 126.111) (end 144.78 129.159) (width 0.25) (layer F.Cu) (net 12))
 (segment (start 147.828 124.333) (end 147.828 126.111) (width 0.25) (layer F.Cu) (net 12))
 (segment (start 147.32 123.825) (end 147.828 124.333) (width 0.25) (layer F.Cu) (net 12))
 (segment (start 144.78 129.159) (end 144.78 129.54) (width 0.25) (layer F.Cu) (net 12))
 (segment (start 147.32 129.54) (end 147.32 128.651) (width 0.25) (layer F.Cu) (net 13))
 (segment (start 147.193 122.555) (end 146.21 122.555) (width 0.25) (layer F.Cu) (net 13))
 (segment (start 148.717 124.079) (end 147.193 122.555) (width 0.25) (layer F.Cu) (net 13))
 (segment (start 148.717 127.254) (end 148.717 124.079) (width 0.25) (layer F.Cu) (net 13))
 (segment (start 147.32 128.651) (end 148.717 127.254) (width 0.25) (layer F.Cu) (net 13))
 (segment (start 152.4 129.54) (end 152.4 128.83) (width 0.25) (layer F.Cu) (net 1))
 (segment (start 152.4 128.83) (end 156.77 124.46) (width 0.25) (layer F.Cu) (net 1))
 (segment (start 155.18 113.03) (end 155.18 123.124) (width 0.25) (layer F.Cu) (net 1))
 (segment (start 155.18 123.124) (end 156.516 124.46) (width 0.25) (layer F.Cu) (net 1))
 (segment (start 154.2288 104.14) (end 154.2288 112.0788) (width 0.25) (layer F.Cu) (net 1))
 (segment (start 154.2288 112.0788) (end 155.18 113.03) (width 0.25) (layer F.Cu) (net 1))
 (segment (start 143.94 102.87) (end 152.9588 102.87) (width 0.25) (layer F.Cu) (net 1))
 (segment (start 152.9588 102.87) (end 154.2288 104.14) (width 0.25) (layer F.Cu) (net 1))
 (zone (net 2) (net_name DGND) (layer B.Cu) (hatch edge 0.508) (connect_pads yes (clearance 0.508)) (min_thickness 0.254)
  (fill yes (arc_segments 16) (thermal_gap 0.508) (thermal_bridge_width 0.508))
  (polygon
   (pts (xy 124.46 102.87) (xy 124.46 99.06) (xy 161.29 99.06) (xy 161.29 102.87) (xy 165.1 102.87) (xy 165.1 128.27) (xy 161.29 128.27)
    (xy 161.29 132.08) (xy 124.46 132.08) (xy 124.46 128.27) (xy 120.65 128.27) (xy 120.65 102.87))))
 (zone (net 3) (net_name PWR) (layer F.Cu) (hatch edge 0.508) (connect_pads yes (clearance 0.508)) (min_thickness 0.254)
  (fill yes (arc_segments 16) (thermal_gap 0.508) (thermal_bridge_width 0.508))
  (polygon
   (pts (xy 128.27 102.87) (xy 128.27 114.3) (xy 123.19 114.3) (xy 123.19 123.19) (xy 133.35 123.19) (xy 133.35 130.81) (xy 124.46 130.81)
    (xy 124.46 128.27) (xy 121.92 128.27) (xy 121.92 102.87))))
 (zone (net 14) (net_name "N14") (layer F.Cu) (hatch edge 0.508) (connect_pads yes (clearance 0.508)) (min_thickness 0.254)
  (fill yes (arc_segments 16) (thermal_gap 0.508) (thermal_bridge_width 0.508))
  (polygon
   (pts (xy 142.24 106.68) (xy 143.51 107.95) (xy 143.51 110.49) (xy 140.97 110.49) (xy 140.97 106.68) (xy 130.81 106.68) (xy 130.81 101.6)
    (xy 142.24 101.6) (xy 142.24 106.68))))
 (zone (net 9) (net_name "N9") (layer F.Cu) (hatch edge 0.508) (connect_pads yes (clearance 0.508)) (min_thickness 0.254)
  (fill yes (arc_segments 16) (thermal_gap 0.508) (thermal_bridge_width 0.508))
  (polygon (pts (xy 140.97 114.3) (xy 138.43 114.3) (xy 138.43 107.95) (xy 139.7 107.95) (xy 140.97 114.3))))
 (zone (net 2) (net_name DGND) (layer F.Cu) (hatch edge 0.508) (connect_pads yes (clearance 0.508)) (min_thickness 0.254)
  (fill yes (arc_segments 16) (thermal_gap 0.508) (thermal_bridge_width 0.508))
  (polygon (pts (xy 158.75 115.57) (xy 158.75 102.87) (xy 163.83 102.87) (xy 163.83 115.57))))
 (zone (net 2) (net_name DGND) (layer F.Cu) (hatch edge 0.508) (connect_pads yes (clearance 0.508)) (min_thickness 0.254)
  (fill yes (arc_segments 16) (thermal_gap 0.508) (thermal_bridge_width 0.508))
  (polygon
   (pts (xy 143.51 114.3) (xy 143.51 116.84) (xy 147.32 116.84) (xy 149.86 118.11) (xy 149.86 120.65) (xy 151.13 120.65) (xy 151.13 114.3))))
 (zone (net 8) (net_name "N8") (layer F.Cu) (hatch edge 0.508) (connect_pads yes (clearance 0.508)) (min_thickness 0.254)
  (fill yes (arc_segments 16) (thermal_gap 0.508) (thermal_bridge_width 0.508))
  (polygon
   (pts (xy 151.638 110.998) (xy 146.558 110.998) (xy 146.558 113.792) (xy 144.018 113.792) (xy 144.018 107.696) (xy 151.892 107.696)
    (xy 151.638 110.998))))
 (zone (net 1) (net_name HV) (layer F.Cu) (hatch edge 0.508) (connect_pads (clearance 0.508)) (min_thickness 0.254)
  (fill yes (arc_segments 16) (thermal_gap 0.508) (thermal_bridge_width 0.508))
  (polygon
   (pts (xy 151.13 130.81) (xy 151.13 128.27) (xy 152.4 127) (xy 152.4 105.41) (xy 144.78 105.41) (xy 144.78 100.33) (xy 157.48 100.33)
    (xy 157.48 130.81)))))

